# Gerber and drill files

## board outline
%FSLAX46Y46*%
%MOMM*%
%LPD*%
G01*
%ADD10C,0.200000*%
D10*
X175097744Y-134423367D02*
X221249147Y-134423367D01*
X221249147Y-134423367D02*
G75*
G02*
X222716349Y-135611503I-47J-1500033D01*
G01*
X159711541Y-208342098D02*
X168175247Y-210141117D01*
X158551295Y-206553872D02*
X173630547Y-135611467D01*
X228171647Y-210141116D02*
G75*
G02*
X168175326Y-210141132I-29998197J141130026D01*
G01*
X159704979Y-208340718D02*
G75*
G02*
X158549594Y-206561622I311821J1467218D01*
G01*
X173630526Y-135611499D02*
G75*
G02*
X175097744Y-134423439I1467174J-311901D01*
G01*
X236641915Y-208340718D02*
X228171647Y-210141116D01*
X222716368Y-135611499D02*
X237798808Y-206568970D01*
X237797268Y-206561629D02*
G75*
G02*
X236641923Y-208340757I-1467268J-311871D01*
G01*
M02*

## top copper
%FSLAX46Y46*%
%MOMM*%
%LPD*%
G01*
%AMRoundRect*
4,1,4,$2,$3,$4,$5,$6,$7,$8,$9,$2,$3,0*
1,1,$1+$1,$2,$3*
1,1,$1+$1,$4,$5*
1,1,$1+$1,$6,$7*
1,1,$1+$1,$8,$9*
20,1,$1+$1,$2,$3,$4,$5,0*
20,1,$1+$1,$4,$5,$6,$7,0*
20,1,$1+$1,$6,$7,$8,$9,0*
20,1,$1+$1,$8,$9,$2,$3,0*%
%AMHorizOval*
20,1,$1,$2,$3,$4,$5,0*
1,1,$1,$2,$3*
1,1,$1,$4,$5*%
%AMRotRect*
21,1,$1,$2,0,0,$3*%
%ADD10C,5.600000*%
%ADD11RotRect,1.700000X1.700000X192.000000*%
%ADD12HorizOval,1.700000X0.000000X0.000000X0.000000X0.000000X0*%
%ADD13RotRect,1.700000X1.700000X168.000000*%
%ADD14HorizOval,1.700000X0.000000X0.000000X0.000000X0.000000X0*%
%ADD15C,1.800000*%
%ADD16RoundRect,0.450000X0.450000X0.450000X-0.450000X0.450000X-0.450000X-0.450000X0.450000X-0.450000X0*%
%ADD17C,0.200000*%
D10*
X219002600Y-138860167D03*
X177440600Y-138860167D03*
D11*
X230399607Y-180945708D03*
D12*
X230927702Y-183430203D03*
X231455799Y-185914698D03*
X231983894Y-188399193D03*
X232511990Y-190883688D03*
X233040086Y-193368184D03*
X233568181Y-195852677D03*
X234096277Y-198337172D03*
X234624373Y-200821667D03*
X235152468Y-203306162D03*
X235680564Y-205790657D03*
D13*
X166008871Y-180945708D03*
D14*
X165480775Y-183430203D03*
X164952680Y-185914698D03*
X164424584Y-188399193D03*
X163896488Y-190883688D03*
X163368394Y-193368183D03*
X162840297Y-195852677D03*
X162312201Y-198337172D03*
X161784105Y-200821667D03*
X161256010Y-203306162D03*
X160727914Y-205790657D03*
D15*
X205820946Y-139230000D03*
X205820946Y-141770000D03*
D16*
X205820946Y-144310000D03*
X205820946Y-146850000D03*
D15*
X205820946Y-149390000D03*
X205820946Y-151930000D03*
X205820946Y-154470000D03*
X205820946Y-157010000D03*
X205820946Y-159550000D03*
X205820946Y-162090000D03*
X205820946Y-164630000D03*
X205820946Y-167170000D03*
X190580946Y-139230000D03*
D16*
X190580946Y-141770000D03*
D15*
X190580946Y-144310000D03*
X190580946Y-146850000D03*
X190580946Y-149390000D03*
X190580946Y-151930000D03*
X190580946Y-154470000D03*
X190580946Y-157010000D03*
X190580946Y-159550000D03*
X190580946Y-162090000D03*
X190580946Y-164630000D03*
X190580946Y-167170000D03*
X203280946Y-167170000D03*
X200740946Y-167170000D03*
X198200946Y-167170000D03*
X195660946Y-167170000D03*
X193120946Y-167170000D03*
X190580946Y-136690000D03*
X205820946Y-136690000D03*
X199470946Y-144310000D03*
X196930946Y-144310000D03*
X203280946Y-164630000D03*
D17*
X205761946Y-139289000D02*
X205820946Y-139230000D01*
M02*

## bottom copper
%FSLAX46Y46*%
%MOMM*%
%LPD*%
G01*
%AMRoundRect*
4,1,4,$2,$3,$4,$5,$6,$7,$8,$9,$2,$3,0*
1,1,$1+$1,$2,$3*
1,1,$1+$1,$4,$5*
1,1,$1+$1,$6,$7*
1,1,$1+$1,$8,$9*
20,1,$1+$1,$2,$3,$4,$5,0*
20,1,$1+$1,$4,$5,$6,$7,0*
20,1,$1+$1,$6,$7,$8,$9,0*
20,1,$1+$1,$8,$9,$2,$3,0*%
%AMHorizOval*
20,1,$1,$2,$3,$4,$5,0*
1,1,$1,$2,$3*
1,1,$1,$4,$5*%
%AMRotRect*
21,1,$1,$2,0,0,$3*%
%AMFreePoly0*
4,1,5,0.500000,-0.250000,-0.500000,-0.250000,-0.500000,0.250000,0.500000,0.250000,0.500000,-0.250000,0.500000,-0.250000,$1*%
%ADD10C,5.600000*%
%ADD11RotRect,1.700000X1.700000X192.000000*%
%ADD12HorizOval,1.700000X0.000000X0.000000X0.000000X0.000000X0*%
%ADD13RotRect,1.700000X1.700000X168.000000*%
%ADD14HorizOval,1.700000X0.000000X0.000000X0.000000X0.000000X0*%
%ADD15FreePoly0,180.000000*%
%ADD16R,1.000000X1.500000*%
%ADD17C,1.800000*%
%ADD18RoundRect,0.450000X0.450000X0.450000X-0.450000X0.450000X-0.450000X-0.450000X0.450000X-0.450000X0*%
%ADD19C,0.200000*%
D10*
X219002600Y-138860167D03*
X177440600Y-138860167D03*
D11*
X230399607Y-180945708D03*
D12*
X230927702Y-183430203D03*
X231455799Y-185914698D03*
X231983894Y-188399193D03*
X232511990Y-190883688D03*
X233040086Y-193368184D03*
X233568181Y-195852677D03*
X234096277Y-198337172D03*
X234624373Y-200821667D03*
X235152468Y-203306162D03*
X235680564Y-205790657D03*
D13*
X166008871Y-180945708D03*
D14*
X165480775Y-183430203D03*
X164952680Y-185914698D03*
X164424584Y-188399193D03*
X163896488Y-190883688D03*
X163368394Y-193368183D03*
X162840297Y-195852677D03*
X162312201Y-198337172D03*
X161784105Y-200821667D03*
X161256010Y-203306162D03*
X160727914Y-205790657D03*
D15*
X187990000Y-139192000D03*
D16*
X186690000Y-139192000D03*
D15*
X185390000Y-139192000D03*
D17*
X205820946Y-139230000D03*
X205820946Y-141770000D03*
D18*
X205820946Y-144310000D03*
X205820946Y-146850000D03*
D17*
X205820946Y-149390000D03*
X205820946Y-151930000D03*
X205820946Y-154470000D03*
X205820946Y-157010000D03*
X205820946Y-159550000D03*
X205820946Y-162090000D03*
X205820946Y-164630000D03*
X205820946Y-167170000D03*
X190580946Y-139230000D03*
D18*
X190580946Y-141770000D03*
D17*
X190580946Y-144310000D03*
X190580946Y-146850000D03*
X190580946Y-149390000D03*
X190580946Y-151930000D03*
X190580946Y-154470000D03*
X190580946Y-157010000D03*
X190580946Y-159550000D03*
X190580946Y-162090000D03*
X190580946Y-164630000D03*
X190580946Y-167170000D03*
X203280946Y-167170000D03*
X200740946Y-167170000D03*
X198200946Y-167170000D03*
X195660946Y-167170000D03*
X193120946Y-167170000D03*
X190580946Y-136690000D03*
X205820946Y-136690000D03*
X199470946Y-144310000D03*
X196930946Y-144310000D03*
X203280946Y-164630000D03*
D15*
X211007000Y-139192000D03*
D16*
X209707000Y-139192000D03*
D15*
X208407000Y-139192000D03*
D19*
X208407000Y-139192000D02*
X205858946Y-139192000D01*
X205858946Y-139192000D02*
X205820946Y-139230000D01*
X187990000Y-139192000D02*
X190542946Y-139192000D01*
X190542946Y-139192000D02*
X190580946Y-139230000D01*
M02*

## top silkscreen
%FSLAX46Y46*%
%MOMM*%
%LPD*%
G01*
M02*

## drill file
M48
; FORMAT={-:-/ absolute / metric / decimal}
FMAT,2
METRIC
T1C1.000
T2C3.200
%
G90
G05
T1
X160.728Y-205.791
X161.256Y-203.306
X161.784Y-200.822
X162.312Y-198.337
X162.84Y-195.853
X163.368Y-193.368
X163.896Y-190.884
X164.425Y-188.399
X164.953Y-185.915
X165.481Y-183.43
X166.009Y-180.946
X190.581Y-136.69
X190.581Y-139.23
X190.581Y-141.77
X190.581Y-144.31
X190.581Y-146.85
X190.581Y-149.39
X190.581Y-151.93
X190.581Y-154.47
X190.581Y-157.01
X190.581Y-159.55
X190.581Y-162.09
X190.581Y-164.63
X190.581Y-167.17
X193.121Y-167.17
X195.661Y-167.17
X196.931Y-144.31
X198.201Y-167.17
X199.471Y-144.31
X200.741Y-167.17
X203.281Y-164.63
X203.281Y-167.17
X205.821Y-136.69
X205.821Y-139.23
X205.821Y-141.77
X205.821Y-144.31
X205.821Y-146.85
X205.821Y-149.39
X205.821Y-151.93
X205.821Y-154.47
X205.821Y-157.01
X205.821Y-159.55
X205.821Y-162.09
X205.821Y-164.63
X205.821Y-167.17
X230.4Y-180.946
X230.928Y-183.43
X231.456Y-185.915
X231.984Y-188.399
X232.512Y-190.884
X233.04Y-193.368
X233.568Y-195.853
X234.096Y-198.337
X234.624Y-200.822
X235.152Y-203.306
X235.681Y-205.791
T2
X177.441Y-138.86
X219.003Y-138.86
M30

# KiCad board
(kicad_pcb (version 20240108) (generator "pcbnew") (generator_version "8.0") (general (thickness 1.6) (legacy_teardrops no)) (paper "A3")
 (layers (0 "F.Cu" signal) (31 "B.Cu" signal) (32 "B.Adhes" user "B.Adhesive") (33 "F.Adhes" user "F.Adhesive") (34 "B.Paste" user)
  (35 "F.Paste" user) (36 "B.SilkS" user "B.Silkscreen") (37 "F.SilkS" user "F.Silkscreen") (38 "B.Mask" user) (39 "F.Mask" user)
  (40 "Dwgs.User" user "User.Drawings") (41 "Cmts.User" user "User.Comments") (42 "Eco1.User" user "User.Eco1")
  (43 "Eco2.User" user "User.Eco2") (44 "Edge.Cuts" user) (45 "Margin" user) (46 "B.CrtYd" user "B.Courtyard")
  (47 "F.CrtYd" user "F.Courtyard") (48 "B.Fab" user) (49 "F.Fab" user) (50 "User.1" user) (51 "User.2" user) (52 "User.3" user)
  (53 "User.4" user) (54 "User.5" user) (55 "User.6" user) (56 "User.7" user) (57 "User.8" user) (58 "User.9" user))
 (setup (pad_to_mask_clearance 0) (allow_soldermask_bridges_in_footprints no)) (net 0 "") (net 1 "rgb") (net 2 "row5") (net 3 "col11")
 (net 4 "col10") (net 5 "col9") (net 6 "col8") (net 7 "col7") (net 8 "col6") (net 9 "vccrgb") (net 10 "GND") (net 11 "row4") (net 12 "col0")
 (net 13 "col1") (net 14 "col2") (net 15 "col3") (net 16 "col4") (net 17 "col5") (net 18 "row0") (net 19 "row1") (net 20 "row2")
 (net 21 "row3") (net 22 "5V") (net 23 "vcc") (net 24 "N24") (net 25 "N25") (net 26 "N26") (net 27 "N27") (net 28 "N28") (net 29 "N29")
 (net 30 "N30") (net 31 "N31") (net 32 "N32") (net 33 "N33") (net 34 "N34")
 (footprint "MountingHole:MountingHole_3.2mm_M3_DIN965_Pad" (layer "F.Cu") (at 219.0026 138.860167)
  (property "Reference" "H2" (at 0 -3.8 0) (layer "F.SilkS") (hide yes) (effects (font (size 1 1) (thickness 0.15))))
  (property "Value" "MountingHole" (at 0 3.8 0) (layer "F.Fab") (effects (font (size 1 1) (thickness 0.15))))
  (pad "1" thru_hole circle (at 0 0) (size 5.6 5.6) (drill 3.2) (layers "*.Cu" "*.Mask") (remove_unused_layers no)))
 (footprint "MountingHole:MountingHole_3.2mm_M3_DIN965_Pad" (layer "F.Cu") (at 177.4406 138.860167)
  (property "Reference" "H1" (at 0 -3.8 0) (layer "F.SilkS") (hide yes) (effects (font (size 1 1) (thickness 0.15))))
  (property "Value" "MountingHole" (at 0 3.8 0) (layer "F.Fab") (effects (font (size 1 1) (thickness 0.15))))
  (pad "1" thru_hole circle (at 0 0) (size 5.6 5.6) (drill 3.2) (layers "*.Cu" "*.Mask") (remove_unused_layers no)))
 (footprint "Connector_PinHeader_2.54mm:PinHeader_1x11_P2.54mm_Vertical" (layer "B.Cu") (at 230.399607 180.945708 -168)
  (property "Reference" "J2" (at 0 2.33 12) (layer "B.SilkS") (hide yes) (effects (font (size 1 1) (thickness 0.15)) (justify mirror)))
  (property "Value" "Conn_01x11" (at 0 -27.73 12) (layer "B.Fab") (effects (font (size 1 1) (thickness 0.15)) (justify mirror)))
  (pad "1" thru_hole rect (at 0 0 192) (size 1.7 1.7) (drill 1) (layers "*.Cu" "*.Mask") (remove_unused_layers no) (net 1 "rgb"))
  (pad "2" thru_hole oval (at 0.000001 -2.54 192) (size 1.7 1.7) (drill 1) (layers "*.Cu" "*.Mask") (remove_unused_layers no) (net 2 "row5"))
  (pad "3" thru_hole oval (at -0.000001 -5.08 192) (size 1.7 1.7) (drill 1) (layers "*.Cu" "*.Mask") (remove_unused_layers no)
   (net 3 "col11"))
  (pad "4" thru_hole oval (at 0 -7.62 192) (size 1.7 1.7) (drill 1) (layers "*.Cu" "*.Mask") (remove_unused_layers no) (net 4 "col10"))
  (pad "5" thru_hole oval (at 0 -10.16 192) (size 1.7 1.7) (drill 1) (layers "*.Cu" "*.Mask") (remove_unused_layers no) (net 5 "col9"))
  (pad "6" thru_hole oval (at 0 -12.700002 192) (size 1.7 1.7) (drill 1) (layers "*.Cu" "*.Mask") (remove_unused_layers no) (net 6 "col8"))
  (pad "7" thru_hole oval (at 0 -15.24 192) (size 1.7 1.7) (drill 1) (layers "*.Cu" "*.Mask") (remove_unused_layers no) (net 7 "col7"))
  (pad "8" thru_hole oval (at 0 -17.78 192) (size 1.7 1.7) (drill 1) (layers "*.Cu" "*.Mask") (remove_unused_layers no) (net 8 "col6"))
  (pad "9" thru_hole oval (at 0 -20.32 192) (size 1.7 1.7) (drill 1) (layers "*.Cu" "*.Mask") (remove_unused_layers no) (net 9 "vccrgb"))
  (pad "10" thru_hole oval (at 0 -22.86 192) (size 1.7 1.7) (drill 1) (layers "*.Cu" "*.Mask") (remove_unused_layers no) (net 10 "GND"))
  (pad "11" thru_hole oval (at 0 -25.4 192) (size 1.7 1.7) (drill 1) (layers "*.Cu" "*.Mask") (remove_unused_layers no) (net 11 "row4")))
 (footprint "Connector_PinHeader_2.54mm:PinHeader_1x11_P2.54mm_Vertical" (layer "B.Cu") (at 166.008871 180.945708 168)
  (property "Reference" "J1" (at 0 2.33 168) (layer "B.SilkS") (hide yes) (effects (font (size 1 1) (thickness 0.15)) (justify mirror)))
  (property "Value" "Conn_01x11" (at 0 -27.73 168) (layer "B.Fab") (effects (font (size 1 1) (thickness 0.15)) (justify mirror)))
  (pad "1" thru_hole rect (at 0 0 168) (size 1.7 1.7) (drill 1) (layers "*.Cu" "*.Mask") (remove_unused_layers no) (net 10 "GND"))
  (pad "2" thru_hole oval (at 0 -2.54 168) (size 1.7 1.7) (drill 1) (layers "*.Cu" "*.Mask") (remove_unused_layers no) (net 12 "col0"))
  (pad "3" thru_hole oval (at 0 -5.08 168) (size 1.7 1.7) (drill 1) (layers "*.Cu" "*.Mask") (remove_unused_layers no) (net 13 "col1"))
  (pad "4" thru_hole oval (at 0 -7.62 168) (size 1.7 1.7) (drill 1) (layers "*.Cu" "*.Mask") (remove_unused_layers no) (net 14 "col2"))
  (pad "5" thru_hole oval (at 0 -10.16 168) (size 1.7 1.7) (drill 1) (layers "*.Cu" "*.Mask") (remove_unused_layers no) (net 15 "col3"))
  (pad "6" thru_hole oval (at -0.000002 -12.7 168) (size 1.7 1.7) (drill 1) (layers "*.Cu" "*.Mask") (remove_unused_layers no)
   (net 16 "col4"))
  (pad "7" thru_hole oval (at 0 -15.24 168) (size 1.7 1.7) (drill 1) (layers "*.Cu" "*.Mask") (remove_unused_layers no) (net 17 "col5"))
  (pad "8" thru_hole oval (at 0 -17.78 168) (size 1.7 1.7) (drill 1) (layers "*.Cu" "*.Mask") (remove_unused_layers no) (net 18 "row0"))
  (pad "9" thru_hole oval (at 0 -20.32 168) (size 1.7 1.7) (drill 1) (layers "*.Cu" "*.Mask") (remove_unused_layers no) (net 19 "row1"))
  (pad "10" thru_hole oval (at 0 -22.86 168) (size 1.7 1.7) (drill 1) (layers "*.Cu" "*.Mask") (remove_unused_layers no) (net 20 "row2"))
  (pad "11" thru_hole oval (at 0 -25.4 168) (size 1.7 1.7) (drill 1) (layers "*.Cu" "*.Mask") (remove_unused_layers no) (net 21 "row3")))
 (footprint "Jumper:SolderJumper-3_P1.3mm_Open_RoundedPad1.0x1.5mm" (layer "B.Cu") (at 186.69 139.192 180)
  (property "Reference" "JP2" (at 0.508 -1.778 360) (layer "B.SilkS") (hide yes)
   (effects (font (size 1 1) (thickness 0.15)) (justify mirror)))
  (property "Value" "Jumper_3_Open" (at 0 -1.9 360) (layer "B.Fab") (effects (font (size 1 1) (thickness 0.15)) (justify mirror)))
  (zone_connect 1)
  (pad "1" smd custom (at -1.3 0 180) (size 1 0.5) (layers "B.Cu" "B.Mask") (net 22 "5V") (zone_connect 2) (thermal_bridge_angle 45)
   (options (clearance outline) (anchor rect)) (primitives))
  (pad "2" smd rect (at 0 0 180) (size 1 1.5) (layers "B.Cu" "B.Mask") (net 9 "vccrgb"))
  (pad "3" smd custom (at 1.3 0 180) (size 1 0.5) (layers "B.Cu" "B.Mask") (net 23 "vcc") (zone_connect 2) (thermal_bridge_angle 45)
   (options (clearance outline) (anchor rect)) (primitives)))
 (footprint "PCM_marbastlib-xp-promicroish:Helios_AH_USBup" (layer "B.Cu") (at 198.200946 153.2 180)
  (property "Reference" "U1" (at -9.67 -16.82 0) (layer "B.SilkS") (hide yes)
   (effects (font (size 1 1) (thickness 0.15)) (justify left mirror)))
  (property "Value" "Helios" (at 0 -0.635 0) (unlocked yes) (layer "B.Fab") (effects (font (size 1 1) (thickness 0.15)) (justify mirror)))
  (pad "1" thru_hole circle (at -7.62 13.97 180) (size 1.8 1.8) (drill 1) (layers "*.Cu" "F.Mask") (remove_unused_layers no) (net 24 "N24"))
  (pad "2" thru_hole circle (at -7.62 11.43 180) (size 1.8 1.8) (drill 1) (layers "*.Cu" "F.Mask") (remove_unused_layers no) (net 3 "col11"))
  (pad "3" thru_hole roundrect (at -7.62 8.89 180) (size 1.8 1.8) (drill 1) (layers "*.Cu" "F.Mask") (remove_unused_layers no)
   (roundrect_rratio 0.25) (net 10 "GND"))
  (pad "4" thru_hole roundrect (at -7.62 6.35 180) (size 1.8 1.8) (drill 1) (layers "*.Cu" "F.Mask") (remove_unused_layers no)
   (roundrect_rratio 0.25) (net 10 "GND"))
  (pad "5" thru_hole circle (at -7.62 3.81 180) (size 1.8 1.8) (drill 1) (layers "*.Cu" "F.Mask") (remove_unused_layers no) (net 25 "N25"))
  (pad "6" thru_hole circle (at -7.62 1.27 180) (size 1.8 1.8) (drill 1) (layers "*.Cu" "F.Mask") (remove_unused_layers no) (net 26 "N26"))
  (pad "7" thru_hole circle (at -7.62 -1.27 180) (size 1.8 1.8) (drill 1) (layers "*.Cu" "F.Mask") (remove_unused_layers no) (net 4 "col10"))
  (pad "8" thru_hole circle (at -7.62 -3.81 180) (size 1.8 1.8) (drill 1) (layers "*.Cu" "F.Mask") (remove_unused_layers no) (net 5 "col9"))
  (pad "9" thru_hole circle (at -7.62 -6.35 180) (size 1.8 1.8) (drill 1) (layers "*.Cu" "F.Mask") (remove_unused_layers no) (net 6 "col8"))
  (pad "10" thru_hole circle (at -7.62 -8.89 180) (size 1.8 1.8) (drill 1) (layers "*.Cu" "F.Mask") (remove_unused_layers no) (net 7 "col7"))
  (pad "11" thru_hole circle (at -7.62 -11.43 180) (size 1.8 1.8) (drill 1) (layers "*.Cu" "F.Mask") (remove_unused_layers no)
   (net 8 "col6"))
  (pad "12" thru_hole circle (at -7.62 -13.97 180) (size 1.8 1.8) (drill 1) (layers "*.Cu" "F.Mask") (remove_unused_layers no)
   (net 11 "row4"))
  (pad "13" thru_hole circle (at 7.62 13.97 180) (size 1.8 1.8) (drill 1) (layers "*.Cu" "F.Mask") (remove_unused_layers no) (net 22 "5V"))
  (pad "14" thru_hole roundrect (at 7.62 11.43 180) (size 1.8 1.8) (drill 1) (layers "*.Cu" "F.Mask") (remove_unused_layers no)
   (roundrect_rratio 0.25) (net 10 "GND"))
  (pad "15" thru_hole circle (at 7.62 8.89 180) (size 1.8 1.8) (drill 1) (layers "*.Cu" "F.Mask") (remove_unused_layers no) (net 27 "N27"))
  (pad "16" thru_hole circle (at 7.62 6.35 180) (size 1.8 1.8) (drill 1) (layers "*.Cu" "F.Mask") (remove_unused_layers no) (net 23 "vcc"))
  (pad "17" thru_hole circle (at 7.62 3.81 180) (size 1.8 1.8) (drill 1) (layers "*.Cu" "F.Mask") (remove_unused_layers no) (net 13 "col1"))
  (pad "18" thru_hole circle (at 7.62 1.27 180) (size 1.8 1.8) (drill 1) (layers "*.Cu" "F.Mask") (remove_unused_layers no) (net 14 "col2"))
  (pad "19" thru_hole circle (at 7.62 -1.27 180) (size 1.8 1.8) (drill 1) (layers "*.Cu" "F.Mask") (remove_unused_layers no) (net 15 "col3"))
  (pad "20" thru_hole circle (at 7.62 -3.81 180) (size 1.8 1.8) (drill 1) (layers "*.Cu" "F.Mask") (remove_unused_layers no) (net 16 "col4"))
  (pad "21" thru_hole circle (at 7.62 -6.35 180) (size 1.8 1.8) (drill 1) (layers "*.Cu" "F.Mask") (remove_unused_layers no) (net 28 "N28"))
  (pad "22" thru_hole circle (at 7.62 -8.89 180) (size 1.8 1.8) (drill 1) (layers "*.Cu" "F.Mask") (remove_unused_layers no) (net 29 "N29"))
  (pad "23" thru_hole circle (at 7.62 -11.43 180) (size 1.8 1.8) (drill 1) (layers "*.Cu" "F.Mask") (remove_unused_layers no) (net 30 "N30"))
  (pad "24" thru_hole circle (at 7.62 -13.97 180) (size 1.8 1.8) (drill 1) (layers "*.Cu" "F.Mask") (remove_unused_layers no) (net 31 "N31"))
  (pad "25" thru_hole circle (at -5.08 -13.97 180) (size 1.8 1.8) (drill 1) (layers "*.Cu" "F.Mask") (remove_unused_layers no)
   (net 21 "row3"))
  (pad "26" thru_hole circle (at -2.54 -13.97 180) (size 1.8 1.8) (drill 1) (layers "*.Cu" "F.Mask") (remove_unused_layers no)
   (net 20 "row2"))
  (pad "27" thru_hole circle (at 0 -13.97 180) (size 1.8 1.8) (drill 1) (layers "*.Cu" "F.Mask") (remove_unused_layers no) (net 19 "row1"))
  (pad "28" thru_hole circle (at 2.54 -13.97 180) (size 1.8 1.8) (drill 1) (layers "*.Cu" "F.Mask") (remove_unused_layers no)
   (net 18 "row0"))
  (pad "29" thru_hole circle (at 5.08 -13.97 180) (size 1.8 1.8) (drill 1) (layers "*.Cu" "F.Mask") (remove_unused_layers no)
   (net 17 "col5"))
  (pad "30" thru_hole circle (at 7.62 16.51 180) (size 1.8 1.8) (drill 1) (layers "*.Cu" "F.Mask") (remove_unused_layers no) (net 12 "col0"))
  (pad "31" thru_hole circle (at -7.62 16.51 180) (size 1.8 1.8) (drill 1) (layers "*.Cu" "F.Mask") (remove_unused_layers no) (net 2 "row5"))
  (pad "32" thru_hole circle (at -1.27 8.89 180) (size 1.8 1.8) (drill 1) (layers "*.Cu" "F.Mask") (remove_unused_layers no) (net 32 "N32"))
  (pad "33" thru_hole circle (at 1.27 8.89 180) (size 1.8 1.8) (drill 1) (layers "*.Cu" "F.Mask") (remove_unused_layers no) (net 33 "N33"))
  (pad "34" thru_hole circle (at -5.08 -11.43 180) (size 1.8 1.8) (drill 1) (layers "*.Cu" "F.Mask") (remove_unused_layers no)
   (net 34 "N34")))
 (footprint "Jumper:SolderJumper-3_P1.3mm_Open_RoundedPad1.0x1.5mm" (layer "B.Cu") (at 209.707 139.192 180)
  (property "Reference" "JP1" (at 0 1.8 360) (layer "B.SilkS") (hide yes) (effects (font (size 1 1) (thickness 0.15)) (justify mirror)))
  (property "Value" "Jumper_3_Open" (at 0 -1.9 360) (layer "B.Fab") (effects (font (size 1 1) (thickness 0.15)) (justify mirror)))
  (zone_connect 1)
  (pad "1" smd custom (at -1.3 0 180) (size 1 0.5) (layers "B.Cu" "B.Mask") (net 34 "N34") (zone_connect 2) (thermal_bridge_angle 45)
   (options (clearance outline) (anchor rect)) (primitives))
  (pad "2" smd rect (at 0 0 180) (size 1 1.5) (layers "B.Cu" "B.Mask") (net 1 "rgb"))
  (pad "3" smd custom (at 1.3 0 180) (size 1 0.5) (layers "B.Cu" "B.Mask") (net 24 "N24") (zone_connect 2) (thermal_bridge_angle 45)
   (options (clearance outline) (anchor rect)) (primitives)))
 (gr_line (start 175.097744 134.423367) (end 221.249147 134.423367) (stroke (width 0.2) (type default)) (layer "Edge.Cuts"))
 (gr_arc (start 221.249147 134.423367) (mid 222.193127 134.757648) (end 222.716368 135.611499) (stroke (width 0.2) (type default))
  (layer "Edge.Cuts"))
 (gr_line (start 159.711541 208.342098) (end 168.175247 210.141117) (stroke (width 0.2) (type default)) (layer "Edge.Cuts"))
 (gr_line (start 158.551295 206.553872) (end 173.630547 135.611467) (stroke (width 0.2) (type default)) (layer "Edge.Cuts"))
 (gr_arc (start 228.171647 210.141116) (mid 198.173487 213.294063) (end 168.175326 210.141133) (stroke (width 0.2) (type default))
  (layer "Edge.Cuts"))
 (gr_arc (start 159.704979 208.340718) (mid 158.75884 207.690455) (end 158.549626 206.561629) (stroke (width 0.2) (type default))
  (layer "Edge.Cuts"))
 (gr_arc (start 173.630526 135.611499) (mid 174.153765 134.757648) (end 175.097744 134.423367) (stroke (width 0.2) (type default))
  (layer "Edge.Cuts"))
 (gr_line (start 236.641915 208.340718) (end 228.171647 210.141116) (stroke (width 0.2) (type default)) (layer "Edge.Cuts"))
 (gr_line (start 222.716368 135.611499) (end 237.798808 206.56897) (stroke (width 0.2) (type default)) (layer "Edge.Cuts"))
 (gr_arc (start 237.797268 206.561629) (mid 237.588038 207.690436) (end 236.641915 208.340718) (stroke (width 0.2) (type default))
  (layer "Edge.Cuts"))
 (segment (start 205.761946 139.289) (end 205.820946 139.23) (width 0.2) (layer "F.Cu") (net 24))
 (segment (start 208.407 139.192) (end 205.858946 139.192) (width 0.2) (layer "B.Cu") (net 24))
 (segment (start 205.858946 139.192) (end 205.820946 139.23) (width 0.2) (layer "B.Cu") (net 24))
 (segment (start 187.99 139.192) (end 190.542946 139.192) (width 0.2) (layer "B.Cu") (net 22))
 (segment (start 190.542946 139.192) (end 190.580946 139.23) (width 0.2) (layer "B.Cu") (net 22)))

